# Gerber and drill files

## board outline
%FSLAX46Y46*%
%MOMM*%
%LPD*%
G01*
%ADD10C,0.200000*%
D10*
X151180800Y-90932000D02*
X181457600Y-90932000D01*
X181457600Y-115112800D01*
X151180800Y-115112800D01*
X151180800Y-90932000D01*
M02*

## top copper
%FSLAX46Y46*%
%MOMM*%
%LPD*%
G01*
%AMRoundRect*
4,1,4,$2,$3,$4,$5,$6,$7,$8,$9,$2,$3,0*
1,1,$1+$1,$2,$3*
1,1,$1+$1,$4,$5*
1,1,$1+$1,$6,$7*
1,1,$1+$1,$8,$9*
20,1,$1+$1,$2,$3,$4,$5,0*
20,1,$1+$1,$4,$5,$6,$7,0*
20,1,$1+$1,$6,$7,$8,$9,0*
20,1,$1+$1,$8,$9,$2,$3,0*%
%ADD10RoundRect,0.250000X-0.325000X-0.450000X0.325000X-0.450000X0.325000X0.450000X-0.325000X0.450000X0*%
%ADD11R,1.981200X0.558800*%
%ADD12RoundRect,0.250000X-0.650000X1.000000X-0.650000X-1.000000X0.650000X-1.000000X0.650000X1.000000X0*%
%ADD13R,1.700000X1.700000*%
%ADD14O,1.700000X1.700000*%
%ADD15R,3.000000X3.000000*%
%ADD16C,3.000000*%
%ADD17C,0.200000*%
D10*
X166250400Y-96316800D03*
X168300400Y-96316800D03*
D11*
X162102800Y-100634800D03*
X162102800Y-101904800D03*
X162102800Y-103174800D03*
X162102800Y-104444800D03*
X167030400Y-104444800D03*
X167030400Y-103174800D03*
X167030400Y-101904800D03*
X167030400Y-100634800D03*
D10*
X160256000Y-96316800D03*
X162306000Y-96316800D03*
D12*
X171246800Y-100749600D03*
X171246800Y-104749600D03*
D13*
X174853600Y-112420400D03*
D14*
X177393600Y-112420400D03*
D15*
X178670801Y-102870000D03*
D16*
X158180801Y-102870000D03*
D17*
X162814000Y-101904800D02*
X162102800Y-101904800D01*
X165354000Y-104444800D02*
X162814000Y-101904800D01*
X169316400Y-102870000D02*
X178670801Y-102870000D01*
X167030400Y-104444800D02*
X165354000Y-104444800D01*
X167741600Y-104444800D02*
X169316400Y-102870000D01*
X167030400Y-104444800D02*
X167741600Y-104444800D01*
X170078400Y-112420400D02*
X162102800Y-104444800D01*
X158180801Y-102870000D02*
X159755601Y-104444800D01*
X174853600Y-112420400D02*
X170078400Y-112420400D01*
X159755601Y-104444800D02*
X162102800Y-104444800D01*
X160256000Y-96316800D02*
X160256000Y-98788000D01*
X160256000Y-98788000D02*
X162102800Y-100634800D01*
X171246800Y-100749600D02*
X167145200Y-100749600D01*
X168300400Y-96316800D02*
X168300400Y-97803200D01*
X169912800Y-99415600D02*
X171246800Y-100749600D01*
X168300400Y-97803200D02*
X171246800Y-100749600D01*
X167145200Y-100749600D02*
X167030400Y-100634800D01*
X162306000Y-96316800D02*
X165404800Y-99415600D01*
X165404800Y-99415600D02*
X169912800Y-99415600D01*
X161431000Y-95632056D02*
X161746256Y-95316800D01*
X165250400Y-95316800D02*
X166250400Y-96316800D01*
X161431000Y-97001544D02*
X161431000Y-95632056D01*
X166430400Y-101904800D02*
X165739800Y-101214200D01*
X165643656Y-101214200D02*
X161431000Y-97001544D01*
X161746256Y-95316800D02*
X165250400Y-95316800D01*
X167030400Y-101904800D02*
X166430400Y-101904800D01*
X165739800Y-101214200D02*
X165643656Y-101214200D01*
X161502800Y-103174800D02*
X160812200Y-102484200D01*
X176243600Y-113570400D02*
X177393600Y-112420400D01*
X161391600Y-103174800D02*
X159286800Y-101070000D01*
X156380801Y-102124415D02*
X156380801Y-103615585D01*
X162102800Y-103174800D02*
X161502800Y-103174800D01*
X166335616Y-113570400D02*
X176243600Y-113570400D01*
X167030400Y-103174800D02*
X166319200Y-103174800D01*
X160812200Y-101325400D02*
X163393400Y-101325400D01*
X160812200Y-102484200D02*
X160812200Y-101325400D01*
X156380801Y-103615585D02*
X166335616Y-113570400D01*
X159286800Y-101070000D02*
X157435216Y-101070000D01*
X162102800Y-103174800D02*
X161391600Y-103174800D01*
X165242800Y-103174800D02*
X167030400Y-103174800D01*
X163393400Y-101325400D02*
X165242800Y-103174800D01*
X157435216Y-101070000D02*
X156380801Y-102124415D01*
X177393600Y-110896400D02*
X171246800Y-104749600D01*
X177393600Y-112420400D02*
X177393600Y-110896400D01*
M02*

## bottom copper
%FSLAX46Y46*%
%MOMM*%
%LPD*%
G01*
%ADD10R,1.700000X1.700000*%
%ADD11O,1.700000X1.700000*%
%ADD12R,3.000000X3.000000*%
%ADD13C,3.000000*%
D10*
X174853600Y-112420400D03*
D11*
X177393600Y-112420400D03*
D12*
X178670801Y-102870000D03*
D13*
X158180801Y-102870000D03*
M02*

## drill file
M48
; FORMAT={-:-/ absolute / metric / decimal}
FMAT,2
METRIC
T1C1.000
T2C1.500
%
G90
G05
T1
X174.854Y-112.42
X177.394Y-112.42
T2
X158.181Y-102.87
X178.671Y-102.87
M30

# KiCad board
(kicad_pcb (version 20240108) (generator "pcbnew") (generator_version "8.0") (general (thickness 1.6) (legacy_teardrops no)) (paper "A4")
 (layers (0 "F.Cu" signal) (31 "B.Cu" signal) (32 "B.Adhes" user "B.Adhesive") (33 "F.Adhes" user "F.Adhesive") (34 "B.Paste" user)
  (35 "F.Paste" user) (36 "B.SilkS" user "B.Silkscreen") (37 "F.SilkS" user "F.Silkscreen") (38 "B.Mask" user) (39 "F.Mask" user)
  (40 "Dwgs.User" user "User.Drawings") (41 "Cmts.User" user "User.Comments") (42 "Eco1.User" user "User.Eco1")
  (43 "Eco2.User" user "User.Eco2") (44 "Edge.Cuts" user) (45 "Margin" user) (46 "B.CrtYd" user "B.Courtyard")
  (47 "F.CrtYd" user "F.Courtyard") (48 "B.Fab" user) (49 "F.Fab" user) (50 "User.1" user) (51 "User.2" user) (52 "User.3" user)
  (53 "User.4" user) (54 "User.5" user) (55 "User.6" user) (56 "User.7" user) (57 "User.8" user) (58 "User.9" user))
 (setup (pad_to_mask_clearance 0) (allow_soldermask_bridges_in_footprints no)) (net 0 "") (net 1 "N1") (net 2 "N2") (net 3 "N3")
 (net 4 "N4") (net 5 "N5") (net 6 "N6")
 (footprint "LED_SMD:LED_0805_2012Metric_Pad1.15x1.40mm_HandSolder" (layer "F.Cu") (at 167.2754 96.3168)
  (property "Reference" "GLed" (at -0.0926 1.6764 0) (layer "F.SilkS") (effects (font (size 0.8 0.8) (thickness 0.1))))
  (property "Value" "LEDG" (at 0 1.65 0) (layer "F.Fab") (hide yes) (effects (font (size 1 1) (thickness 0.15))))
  (pad "1" smd roundrect (at -1.025 0) (size 1.15 1.4) (layers "F.Cu" "F.Paste" "F.Mask") (roundrect_rratio 0.217391) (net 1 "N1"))
  (pad "2" smd roundrect (at 1.025 0) (size 1.15 1.4) (layers "F.Cu" "F.Paste" "F.Mask") (roundrect_rratio 0.217391) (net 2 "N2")))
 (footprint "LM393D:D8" (layer "F.Cu") (at 164.5666 102.5398)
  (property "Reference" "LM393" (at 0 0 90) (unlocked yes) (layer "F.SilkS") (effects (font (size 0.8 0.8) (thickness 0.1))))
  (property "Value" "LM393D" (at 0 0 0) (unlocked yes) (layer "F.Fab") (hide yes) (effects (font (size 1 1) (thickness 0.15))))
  (pad "1" smd rect (at -2.4638 -1.905) (size 1.9812 0.5588) (layers "F.Cu" "F.Paste" "F.Mask") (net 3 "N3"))
  (pad "2" smd rect (at -2.4638 -0.635) (size 1.9812 0.5588) (layers "F.Cu" "F.Paste" "F.Mask") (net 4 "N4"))
  (pad "3" smd rect (at -2.4638 0.635) (size 1.9812 0.5588) (layers "F.Cu" "F.Paste" "F.Mask") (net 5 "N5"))
  (pad "4" smd rect (at -2.4638 1.905) (size 1.9812 0.5588) (layers "F.Cu" "F.Paste" "F.Mask") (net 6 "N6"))
  (pad "5" smd rect (at 2.4638 1.905) (size 1.9812 0.5588) (layers "F.Cu" "F.Paste" "F.Mask") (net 4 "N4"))
  (pad "6" smd rect (at 2.4638 0.635) (size 1.9812 0.5588) (layers "F.Cu" "F.Paste" "F.Mask") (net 5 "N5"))
  (pad "7" smd rect (at 2.4638 -0.635) (size 1.9812 0.5588) (layers "F.Cu" "F.Paste" "F.Mask") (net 1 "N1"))
  (pad "8" smd rect (at 2.4638 -1.905) (size 1.9812 0.5588) (layers "F.Cu" "F.Paste" "F.Mask") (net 2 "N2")))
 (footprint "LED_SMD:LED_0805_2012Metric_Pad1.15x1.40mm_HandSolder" (layer "F.Cu") (at 161.281 96.3168)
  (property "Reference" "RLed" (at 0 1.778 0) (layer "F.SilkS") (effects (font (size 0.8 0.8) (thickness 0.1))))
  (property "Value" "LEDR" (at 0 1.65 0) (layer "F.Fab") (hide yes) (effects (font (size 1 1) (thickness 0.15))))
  (pad "1" smd roundrect (at -1.025 0) (size 1.15 1.4) (layers "F.Cu" "F.Paste" "F.Mask") (roundrect_rratio 0.217391) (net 3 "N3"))
  (pad "2" smd roundrect (at 1.025 0) (size 1.15 1.4) (layers "F.Cu" "F.Paste" "F.Mask") (roundrect_rratio 0.217391) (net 2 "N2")))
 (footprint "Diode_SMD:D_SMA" (layer "F.Cu") (at 171.2468 102.7496 -90)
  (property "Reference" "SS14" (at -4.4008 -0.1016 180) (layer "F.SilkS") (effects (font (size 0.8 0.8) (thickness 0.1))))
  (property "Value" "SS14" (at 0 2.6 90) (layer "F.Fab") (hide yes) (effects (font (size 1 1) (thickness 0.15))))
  (pad "1" smd roundrect (at -2 0 270) (size 2.5 1.8) (layers "F.Cu" "F.Paste" "F.Mask") (roundrect_rratio 0.1388888889) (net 2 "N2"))
  (pad "2" smd roundrect (at 2 0 270) (size 2.5 1.8) (layers "F.Cu" "F.Paste" "F.Mask") (roundrect_rratio 0.1388888889) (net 5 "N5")))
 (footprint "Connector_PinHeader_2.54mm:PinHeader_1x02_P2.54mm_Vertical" (layer "F.Cu") (at 174.8536 112.4204 90)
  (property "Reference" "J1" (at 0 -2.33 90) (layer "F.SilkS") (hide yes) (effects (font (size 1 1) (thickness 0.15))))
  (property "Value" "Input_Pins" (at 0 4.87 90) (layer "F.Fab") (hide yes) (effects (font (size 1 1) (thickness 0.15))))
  (pad "1" thru_hole rect (at 0 0 90) (size 1.7 1.7) (drill 1) (layers "*.Cu" "*.Mask") (remove_unused_layers no) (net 6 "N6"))
  (pad "2" thru_hole oval (at 0 2.54 90) (size 1.7 1.7) (drill 1) (layers "*.Cu" "*.Mask") (remove_unused_layers no) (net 5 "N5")))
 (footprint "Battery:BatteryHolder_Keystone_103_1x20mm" (layer "B.Cu") (at 178.670801 102.87 180)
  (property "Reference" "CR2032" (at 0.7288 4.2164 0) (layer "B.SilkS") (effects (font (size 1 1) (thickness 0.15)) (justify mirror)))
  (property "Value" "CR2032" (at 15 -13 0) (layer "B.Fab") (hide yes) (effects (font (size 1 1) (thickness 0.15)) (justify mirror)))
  (pad "1" thru_hole rect (at 0 0 180) (size 3 3) (drill 1.5) (layers "*.Cu" "*.Mask") (remove_unused_layers no) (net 4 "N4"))
  (pad "2" thru_hole circle (at 20.49 0 180) (size 3 3) (drill 1.5) (layers "*.Cu" "*.Mask") (remove_unused_layers no) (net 6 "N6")))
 (gr_rect (start 151.1808 90.932) (end 181.4576 115.1128) (stroke (width 0.2) (type default)) (fill none) (layer "Edge.Cuts"))
 (segment (start 162.814 101.9048) (end 162.1028 101.9048) (width 0.2) (layer "F.Cu") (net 4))
 (segment (start 165.354 104.4448) (end 162.814 101.9048) (width 0.2) (layer "F.Cu") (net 4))
 (segment (start 169.3164 102.87) (end 178.670801 102.87) (width 0.2) (layer "F.Cu") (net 4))
 (segment (start 167.0304 104.4448) (end 165.354 104.4448) (width 0.2) (layer "F.Cu") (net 4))
 (segment (start 167.7416 104.4448) (end 169.3164 102.87) (width 0.2) (layer "F.Cu") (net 4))
 (segment (start 167.0304 104.4448) (end 167.7416 104.4448) (width 0.2) (layer "F.Cu") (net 4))
 (segment (start 170.0784 112.4204) (end 162.1028 104.4448) (width 0.2) (layer "F.Cu") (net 6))
 (segment (start 158.180801 102.87) (end 159.755601 104.4448) (width 0.2) (layer "F.Cu") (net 6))
 (segment (start 174.8536 112.4204) (end 170.0784 112.4204) (width 0.2) (layer "F.Cu") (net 6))
 (segment (start 159.755601 104.4448) (end 162.1028 104.4448) (width 0.2) (layer "F.Cu") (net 6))
 (segment (start 160.256 96.3168) (end 160.256 98.788) (width 0.2) (layer "F.Cu") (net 3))
 (segment (start 160.256 98.788) (end 162.1028 100.6348) (width 0.2) (layer "F.Cu") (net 3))
 (segment (start 171.2468 100.7496) (end 167.1452 100.7496) (width 0.2) (layer "F.Cu") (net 2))
 (segment (start 168.3004 96.3168) (end 168.3004 97.8032) (width 0.2) (layer "F.Cu") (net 2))
 (segment (start 169.9128 99.4156) (end 171.2468 100.7496) (width 0.2) (layer "F.Cu") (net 2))
 (segment (start 168.3004 97.8032) (end 171.2468 100.7496) (width 0.2) (layer "F.Cu") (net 2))
 (segment (start 167.1452 100.7496) (end 167.0304 100.6348) (width 0.2) (layer "F.Cu") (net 2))
 (segment (start 162.306 96.3168) (end 165.4048 99.4156) (width 0.2) (layer "F.Cu") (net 2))
 (segment (start 165.4048 99.4156) (end 169.9128 99.4156) (width 0.2) (layer "F.Cu") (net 2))
 (segment (start 161.431 95.632056) (end 161.746256 95.3168) (width 0.2) (layer "F.Cu") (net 1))
 (segment (start 165.2504 95.3168) (end 166.2504 96.3168) (width 0.2) (layer "F.Cu") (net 1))
 (segment (start 161.431 97.001544) (end 161.431 95.632056) (width 0.2) (layer "F.Cu") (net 1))
 (segment (start 166.4304 101.9048) (end 165.7398 101.2142) (width 0.2) (layer "F.Cu") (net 1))
 (segment (start 165.643656 101.2142) (end 161.431 97.001544) (width 0.2) (layer "F.Cu") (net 1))
 (segment (start 161.746256 95.3168) (end 165.2504 95.3168) (width 0.2) (layer "F.Cu") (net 1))
 (segment (start 167.0304 101.9048) (end 166.4304 101.9048) (width 0.2) (layer "F.Cu") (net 1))
 (segment (start 165.7398 101.2142) (end 165.643656 101.2142) (width 0.2) (layer "F.Cu") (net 1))
 (segment (start 161.5028 103.1748) (end 160.8122 102.4842) (width 0.2) (layer "F.Cu") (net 5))
 (segment (start 176.2436 113.5704) (end 177.3936 112.4204) (width 0.2) (layer "F.Cu") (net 5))
 (segment (start 161.3916 103.1748) (end 159.2868 101.07) (width 0.2) (layer "F.Cu") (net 5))
 (segment (start 156.380801 102.124415) (end 156.380801 103.615585) (width 0.2) (layer "F.Cu") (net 5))
 (segment (start 162.1028 103.1748) (end 161.5028 103.1748) (width 0.2) (layer "F.Cu") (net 5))
 (segment (start 166.335616 113.5704) (end 176.2436 113.5704) (width 0.2) (layer "F.Cu") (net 5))
 (segment (start 167.0304 103.1748) (end 166.3192 103.1748) (width 0.2) (layer "F.Cu") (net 5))
 (segment (start 160.8122 101.3254) (end 163.3934 101.3254) (width 0.2) (layer "F.Cu") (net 5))
 (segment (start 160.8122 102.4842) (end 160.8122 101.3254) (width 0.2) (layer "F.Cu") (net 5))
 (segment (start 156.380801 103.615585) (end 166.335616 113.5704) (width 0.2) (layer "F.Cu") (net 5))
 (segment (start 159.2868 101.07) (end 157.435216 101.07) (width 0.2) (layer "F.Cu") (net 5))
 (segment (start 162.1028 103.1748) (end 161.3916 103.1748) (width 0.2) (layer "F.Cu") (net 5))
 (segment (start 165.2428 103.1748) (end 167.0304 103.1748) (width 0.2) (layer "F.Cu") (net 5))
 (segment (start 163.3934 101.3254) (end 165.2428 103.1748) (width 0.2) (layer "F.Cu") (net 5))
 (segment (start 157.435216 101.07) (end 156.380801 102.124415) (width 0.2) (layer "F.Cu") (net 5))
 (segment (start 177.3936 110.8964) (end 171.2468 104.7496) (width 0.2) (layer "F.Cu") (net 5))
 (segment (start 177.3936 112.4204) (end 177.3936 110.8964) (width 0.2) (layer "F.Cu") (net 5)))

